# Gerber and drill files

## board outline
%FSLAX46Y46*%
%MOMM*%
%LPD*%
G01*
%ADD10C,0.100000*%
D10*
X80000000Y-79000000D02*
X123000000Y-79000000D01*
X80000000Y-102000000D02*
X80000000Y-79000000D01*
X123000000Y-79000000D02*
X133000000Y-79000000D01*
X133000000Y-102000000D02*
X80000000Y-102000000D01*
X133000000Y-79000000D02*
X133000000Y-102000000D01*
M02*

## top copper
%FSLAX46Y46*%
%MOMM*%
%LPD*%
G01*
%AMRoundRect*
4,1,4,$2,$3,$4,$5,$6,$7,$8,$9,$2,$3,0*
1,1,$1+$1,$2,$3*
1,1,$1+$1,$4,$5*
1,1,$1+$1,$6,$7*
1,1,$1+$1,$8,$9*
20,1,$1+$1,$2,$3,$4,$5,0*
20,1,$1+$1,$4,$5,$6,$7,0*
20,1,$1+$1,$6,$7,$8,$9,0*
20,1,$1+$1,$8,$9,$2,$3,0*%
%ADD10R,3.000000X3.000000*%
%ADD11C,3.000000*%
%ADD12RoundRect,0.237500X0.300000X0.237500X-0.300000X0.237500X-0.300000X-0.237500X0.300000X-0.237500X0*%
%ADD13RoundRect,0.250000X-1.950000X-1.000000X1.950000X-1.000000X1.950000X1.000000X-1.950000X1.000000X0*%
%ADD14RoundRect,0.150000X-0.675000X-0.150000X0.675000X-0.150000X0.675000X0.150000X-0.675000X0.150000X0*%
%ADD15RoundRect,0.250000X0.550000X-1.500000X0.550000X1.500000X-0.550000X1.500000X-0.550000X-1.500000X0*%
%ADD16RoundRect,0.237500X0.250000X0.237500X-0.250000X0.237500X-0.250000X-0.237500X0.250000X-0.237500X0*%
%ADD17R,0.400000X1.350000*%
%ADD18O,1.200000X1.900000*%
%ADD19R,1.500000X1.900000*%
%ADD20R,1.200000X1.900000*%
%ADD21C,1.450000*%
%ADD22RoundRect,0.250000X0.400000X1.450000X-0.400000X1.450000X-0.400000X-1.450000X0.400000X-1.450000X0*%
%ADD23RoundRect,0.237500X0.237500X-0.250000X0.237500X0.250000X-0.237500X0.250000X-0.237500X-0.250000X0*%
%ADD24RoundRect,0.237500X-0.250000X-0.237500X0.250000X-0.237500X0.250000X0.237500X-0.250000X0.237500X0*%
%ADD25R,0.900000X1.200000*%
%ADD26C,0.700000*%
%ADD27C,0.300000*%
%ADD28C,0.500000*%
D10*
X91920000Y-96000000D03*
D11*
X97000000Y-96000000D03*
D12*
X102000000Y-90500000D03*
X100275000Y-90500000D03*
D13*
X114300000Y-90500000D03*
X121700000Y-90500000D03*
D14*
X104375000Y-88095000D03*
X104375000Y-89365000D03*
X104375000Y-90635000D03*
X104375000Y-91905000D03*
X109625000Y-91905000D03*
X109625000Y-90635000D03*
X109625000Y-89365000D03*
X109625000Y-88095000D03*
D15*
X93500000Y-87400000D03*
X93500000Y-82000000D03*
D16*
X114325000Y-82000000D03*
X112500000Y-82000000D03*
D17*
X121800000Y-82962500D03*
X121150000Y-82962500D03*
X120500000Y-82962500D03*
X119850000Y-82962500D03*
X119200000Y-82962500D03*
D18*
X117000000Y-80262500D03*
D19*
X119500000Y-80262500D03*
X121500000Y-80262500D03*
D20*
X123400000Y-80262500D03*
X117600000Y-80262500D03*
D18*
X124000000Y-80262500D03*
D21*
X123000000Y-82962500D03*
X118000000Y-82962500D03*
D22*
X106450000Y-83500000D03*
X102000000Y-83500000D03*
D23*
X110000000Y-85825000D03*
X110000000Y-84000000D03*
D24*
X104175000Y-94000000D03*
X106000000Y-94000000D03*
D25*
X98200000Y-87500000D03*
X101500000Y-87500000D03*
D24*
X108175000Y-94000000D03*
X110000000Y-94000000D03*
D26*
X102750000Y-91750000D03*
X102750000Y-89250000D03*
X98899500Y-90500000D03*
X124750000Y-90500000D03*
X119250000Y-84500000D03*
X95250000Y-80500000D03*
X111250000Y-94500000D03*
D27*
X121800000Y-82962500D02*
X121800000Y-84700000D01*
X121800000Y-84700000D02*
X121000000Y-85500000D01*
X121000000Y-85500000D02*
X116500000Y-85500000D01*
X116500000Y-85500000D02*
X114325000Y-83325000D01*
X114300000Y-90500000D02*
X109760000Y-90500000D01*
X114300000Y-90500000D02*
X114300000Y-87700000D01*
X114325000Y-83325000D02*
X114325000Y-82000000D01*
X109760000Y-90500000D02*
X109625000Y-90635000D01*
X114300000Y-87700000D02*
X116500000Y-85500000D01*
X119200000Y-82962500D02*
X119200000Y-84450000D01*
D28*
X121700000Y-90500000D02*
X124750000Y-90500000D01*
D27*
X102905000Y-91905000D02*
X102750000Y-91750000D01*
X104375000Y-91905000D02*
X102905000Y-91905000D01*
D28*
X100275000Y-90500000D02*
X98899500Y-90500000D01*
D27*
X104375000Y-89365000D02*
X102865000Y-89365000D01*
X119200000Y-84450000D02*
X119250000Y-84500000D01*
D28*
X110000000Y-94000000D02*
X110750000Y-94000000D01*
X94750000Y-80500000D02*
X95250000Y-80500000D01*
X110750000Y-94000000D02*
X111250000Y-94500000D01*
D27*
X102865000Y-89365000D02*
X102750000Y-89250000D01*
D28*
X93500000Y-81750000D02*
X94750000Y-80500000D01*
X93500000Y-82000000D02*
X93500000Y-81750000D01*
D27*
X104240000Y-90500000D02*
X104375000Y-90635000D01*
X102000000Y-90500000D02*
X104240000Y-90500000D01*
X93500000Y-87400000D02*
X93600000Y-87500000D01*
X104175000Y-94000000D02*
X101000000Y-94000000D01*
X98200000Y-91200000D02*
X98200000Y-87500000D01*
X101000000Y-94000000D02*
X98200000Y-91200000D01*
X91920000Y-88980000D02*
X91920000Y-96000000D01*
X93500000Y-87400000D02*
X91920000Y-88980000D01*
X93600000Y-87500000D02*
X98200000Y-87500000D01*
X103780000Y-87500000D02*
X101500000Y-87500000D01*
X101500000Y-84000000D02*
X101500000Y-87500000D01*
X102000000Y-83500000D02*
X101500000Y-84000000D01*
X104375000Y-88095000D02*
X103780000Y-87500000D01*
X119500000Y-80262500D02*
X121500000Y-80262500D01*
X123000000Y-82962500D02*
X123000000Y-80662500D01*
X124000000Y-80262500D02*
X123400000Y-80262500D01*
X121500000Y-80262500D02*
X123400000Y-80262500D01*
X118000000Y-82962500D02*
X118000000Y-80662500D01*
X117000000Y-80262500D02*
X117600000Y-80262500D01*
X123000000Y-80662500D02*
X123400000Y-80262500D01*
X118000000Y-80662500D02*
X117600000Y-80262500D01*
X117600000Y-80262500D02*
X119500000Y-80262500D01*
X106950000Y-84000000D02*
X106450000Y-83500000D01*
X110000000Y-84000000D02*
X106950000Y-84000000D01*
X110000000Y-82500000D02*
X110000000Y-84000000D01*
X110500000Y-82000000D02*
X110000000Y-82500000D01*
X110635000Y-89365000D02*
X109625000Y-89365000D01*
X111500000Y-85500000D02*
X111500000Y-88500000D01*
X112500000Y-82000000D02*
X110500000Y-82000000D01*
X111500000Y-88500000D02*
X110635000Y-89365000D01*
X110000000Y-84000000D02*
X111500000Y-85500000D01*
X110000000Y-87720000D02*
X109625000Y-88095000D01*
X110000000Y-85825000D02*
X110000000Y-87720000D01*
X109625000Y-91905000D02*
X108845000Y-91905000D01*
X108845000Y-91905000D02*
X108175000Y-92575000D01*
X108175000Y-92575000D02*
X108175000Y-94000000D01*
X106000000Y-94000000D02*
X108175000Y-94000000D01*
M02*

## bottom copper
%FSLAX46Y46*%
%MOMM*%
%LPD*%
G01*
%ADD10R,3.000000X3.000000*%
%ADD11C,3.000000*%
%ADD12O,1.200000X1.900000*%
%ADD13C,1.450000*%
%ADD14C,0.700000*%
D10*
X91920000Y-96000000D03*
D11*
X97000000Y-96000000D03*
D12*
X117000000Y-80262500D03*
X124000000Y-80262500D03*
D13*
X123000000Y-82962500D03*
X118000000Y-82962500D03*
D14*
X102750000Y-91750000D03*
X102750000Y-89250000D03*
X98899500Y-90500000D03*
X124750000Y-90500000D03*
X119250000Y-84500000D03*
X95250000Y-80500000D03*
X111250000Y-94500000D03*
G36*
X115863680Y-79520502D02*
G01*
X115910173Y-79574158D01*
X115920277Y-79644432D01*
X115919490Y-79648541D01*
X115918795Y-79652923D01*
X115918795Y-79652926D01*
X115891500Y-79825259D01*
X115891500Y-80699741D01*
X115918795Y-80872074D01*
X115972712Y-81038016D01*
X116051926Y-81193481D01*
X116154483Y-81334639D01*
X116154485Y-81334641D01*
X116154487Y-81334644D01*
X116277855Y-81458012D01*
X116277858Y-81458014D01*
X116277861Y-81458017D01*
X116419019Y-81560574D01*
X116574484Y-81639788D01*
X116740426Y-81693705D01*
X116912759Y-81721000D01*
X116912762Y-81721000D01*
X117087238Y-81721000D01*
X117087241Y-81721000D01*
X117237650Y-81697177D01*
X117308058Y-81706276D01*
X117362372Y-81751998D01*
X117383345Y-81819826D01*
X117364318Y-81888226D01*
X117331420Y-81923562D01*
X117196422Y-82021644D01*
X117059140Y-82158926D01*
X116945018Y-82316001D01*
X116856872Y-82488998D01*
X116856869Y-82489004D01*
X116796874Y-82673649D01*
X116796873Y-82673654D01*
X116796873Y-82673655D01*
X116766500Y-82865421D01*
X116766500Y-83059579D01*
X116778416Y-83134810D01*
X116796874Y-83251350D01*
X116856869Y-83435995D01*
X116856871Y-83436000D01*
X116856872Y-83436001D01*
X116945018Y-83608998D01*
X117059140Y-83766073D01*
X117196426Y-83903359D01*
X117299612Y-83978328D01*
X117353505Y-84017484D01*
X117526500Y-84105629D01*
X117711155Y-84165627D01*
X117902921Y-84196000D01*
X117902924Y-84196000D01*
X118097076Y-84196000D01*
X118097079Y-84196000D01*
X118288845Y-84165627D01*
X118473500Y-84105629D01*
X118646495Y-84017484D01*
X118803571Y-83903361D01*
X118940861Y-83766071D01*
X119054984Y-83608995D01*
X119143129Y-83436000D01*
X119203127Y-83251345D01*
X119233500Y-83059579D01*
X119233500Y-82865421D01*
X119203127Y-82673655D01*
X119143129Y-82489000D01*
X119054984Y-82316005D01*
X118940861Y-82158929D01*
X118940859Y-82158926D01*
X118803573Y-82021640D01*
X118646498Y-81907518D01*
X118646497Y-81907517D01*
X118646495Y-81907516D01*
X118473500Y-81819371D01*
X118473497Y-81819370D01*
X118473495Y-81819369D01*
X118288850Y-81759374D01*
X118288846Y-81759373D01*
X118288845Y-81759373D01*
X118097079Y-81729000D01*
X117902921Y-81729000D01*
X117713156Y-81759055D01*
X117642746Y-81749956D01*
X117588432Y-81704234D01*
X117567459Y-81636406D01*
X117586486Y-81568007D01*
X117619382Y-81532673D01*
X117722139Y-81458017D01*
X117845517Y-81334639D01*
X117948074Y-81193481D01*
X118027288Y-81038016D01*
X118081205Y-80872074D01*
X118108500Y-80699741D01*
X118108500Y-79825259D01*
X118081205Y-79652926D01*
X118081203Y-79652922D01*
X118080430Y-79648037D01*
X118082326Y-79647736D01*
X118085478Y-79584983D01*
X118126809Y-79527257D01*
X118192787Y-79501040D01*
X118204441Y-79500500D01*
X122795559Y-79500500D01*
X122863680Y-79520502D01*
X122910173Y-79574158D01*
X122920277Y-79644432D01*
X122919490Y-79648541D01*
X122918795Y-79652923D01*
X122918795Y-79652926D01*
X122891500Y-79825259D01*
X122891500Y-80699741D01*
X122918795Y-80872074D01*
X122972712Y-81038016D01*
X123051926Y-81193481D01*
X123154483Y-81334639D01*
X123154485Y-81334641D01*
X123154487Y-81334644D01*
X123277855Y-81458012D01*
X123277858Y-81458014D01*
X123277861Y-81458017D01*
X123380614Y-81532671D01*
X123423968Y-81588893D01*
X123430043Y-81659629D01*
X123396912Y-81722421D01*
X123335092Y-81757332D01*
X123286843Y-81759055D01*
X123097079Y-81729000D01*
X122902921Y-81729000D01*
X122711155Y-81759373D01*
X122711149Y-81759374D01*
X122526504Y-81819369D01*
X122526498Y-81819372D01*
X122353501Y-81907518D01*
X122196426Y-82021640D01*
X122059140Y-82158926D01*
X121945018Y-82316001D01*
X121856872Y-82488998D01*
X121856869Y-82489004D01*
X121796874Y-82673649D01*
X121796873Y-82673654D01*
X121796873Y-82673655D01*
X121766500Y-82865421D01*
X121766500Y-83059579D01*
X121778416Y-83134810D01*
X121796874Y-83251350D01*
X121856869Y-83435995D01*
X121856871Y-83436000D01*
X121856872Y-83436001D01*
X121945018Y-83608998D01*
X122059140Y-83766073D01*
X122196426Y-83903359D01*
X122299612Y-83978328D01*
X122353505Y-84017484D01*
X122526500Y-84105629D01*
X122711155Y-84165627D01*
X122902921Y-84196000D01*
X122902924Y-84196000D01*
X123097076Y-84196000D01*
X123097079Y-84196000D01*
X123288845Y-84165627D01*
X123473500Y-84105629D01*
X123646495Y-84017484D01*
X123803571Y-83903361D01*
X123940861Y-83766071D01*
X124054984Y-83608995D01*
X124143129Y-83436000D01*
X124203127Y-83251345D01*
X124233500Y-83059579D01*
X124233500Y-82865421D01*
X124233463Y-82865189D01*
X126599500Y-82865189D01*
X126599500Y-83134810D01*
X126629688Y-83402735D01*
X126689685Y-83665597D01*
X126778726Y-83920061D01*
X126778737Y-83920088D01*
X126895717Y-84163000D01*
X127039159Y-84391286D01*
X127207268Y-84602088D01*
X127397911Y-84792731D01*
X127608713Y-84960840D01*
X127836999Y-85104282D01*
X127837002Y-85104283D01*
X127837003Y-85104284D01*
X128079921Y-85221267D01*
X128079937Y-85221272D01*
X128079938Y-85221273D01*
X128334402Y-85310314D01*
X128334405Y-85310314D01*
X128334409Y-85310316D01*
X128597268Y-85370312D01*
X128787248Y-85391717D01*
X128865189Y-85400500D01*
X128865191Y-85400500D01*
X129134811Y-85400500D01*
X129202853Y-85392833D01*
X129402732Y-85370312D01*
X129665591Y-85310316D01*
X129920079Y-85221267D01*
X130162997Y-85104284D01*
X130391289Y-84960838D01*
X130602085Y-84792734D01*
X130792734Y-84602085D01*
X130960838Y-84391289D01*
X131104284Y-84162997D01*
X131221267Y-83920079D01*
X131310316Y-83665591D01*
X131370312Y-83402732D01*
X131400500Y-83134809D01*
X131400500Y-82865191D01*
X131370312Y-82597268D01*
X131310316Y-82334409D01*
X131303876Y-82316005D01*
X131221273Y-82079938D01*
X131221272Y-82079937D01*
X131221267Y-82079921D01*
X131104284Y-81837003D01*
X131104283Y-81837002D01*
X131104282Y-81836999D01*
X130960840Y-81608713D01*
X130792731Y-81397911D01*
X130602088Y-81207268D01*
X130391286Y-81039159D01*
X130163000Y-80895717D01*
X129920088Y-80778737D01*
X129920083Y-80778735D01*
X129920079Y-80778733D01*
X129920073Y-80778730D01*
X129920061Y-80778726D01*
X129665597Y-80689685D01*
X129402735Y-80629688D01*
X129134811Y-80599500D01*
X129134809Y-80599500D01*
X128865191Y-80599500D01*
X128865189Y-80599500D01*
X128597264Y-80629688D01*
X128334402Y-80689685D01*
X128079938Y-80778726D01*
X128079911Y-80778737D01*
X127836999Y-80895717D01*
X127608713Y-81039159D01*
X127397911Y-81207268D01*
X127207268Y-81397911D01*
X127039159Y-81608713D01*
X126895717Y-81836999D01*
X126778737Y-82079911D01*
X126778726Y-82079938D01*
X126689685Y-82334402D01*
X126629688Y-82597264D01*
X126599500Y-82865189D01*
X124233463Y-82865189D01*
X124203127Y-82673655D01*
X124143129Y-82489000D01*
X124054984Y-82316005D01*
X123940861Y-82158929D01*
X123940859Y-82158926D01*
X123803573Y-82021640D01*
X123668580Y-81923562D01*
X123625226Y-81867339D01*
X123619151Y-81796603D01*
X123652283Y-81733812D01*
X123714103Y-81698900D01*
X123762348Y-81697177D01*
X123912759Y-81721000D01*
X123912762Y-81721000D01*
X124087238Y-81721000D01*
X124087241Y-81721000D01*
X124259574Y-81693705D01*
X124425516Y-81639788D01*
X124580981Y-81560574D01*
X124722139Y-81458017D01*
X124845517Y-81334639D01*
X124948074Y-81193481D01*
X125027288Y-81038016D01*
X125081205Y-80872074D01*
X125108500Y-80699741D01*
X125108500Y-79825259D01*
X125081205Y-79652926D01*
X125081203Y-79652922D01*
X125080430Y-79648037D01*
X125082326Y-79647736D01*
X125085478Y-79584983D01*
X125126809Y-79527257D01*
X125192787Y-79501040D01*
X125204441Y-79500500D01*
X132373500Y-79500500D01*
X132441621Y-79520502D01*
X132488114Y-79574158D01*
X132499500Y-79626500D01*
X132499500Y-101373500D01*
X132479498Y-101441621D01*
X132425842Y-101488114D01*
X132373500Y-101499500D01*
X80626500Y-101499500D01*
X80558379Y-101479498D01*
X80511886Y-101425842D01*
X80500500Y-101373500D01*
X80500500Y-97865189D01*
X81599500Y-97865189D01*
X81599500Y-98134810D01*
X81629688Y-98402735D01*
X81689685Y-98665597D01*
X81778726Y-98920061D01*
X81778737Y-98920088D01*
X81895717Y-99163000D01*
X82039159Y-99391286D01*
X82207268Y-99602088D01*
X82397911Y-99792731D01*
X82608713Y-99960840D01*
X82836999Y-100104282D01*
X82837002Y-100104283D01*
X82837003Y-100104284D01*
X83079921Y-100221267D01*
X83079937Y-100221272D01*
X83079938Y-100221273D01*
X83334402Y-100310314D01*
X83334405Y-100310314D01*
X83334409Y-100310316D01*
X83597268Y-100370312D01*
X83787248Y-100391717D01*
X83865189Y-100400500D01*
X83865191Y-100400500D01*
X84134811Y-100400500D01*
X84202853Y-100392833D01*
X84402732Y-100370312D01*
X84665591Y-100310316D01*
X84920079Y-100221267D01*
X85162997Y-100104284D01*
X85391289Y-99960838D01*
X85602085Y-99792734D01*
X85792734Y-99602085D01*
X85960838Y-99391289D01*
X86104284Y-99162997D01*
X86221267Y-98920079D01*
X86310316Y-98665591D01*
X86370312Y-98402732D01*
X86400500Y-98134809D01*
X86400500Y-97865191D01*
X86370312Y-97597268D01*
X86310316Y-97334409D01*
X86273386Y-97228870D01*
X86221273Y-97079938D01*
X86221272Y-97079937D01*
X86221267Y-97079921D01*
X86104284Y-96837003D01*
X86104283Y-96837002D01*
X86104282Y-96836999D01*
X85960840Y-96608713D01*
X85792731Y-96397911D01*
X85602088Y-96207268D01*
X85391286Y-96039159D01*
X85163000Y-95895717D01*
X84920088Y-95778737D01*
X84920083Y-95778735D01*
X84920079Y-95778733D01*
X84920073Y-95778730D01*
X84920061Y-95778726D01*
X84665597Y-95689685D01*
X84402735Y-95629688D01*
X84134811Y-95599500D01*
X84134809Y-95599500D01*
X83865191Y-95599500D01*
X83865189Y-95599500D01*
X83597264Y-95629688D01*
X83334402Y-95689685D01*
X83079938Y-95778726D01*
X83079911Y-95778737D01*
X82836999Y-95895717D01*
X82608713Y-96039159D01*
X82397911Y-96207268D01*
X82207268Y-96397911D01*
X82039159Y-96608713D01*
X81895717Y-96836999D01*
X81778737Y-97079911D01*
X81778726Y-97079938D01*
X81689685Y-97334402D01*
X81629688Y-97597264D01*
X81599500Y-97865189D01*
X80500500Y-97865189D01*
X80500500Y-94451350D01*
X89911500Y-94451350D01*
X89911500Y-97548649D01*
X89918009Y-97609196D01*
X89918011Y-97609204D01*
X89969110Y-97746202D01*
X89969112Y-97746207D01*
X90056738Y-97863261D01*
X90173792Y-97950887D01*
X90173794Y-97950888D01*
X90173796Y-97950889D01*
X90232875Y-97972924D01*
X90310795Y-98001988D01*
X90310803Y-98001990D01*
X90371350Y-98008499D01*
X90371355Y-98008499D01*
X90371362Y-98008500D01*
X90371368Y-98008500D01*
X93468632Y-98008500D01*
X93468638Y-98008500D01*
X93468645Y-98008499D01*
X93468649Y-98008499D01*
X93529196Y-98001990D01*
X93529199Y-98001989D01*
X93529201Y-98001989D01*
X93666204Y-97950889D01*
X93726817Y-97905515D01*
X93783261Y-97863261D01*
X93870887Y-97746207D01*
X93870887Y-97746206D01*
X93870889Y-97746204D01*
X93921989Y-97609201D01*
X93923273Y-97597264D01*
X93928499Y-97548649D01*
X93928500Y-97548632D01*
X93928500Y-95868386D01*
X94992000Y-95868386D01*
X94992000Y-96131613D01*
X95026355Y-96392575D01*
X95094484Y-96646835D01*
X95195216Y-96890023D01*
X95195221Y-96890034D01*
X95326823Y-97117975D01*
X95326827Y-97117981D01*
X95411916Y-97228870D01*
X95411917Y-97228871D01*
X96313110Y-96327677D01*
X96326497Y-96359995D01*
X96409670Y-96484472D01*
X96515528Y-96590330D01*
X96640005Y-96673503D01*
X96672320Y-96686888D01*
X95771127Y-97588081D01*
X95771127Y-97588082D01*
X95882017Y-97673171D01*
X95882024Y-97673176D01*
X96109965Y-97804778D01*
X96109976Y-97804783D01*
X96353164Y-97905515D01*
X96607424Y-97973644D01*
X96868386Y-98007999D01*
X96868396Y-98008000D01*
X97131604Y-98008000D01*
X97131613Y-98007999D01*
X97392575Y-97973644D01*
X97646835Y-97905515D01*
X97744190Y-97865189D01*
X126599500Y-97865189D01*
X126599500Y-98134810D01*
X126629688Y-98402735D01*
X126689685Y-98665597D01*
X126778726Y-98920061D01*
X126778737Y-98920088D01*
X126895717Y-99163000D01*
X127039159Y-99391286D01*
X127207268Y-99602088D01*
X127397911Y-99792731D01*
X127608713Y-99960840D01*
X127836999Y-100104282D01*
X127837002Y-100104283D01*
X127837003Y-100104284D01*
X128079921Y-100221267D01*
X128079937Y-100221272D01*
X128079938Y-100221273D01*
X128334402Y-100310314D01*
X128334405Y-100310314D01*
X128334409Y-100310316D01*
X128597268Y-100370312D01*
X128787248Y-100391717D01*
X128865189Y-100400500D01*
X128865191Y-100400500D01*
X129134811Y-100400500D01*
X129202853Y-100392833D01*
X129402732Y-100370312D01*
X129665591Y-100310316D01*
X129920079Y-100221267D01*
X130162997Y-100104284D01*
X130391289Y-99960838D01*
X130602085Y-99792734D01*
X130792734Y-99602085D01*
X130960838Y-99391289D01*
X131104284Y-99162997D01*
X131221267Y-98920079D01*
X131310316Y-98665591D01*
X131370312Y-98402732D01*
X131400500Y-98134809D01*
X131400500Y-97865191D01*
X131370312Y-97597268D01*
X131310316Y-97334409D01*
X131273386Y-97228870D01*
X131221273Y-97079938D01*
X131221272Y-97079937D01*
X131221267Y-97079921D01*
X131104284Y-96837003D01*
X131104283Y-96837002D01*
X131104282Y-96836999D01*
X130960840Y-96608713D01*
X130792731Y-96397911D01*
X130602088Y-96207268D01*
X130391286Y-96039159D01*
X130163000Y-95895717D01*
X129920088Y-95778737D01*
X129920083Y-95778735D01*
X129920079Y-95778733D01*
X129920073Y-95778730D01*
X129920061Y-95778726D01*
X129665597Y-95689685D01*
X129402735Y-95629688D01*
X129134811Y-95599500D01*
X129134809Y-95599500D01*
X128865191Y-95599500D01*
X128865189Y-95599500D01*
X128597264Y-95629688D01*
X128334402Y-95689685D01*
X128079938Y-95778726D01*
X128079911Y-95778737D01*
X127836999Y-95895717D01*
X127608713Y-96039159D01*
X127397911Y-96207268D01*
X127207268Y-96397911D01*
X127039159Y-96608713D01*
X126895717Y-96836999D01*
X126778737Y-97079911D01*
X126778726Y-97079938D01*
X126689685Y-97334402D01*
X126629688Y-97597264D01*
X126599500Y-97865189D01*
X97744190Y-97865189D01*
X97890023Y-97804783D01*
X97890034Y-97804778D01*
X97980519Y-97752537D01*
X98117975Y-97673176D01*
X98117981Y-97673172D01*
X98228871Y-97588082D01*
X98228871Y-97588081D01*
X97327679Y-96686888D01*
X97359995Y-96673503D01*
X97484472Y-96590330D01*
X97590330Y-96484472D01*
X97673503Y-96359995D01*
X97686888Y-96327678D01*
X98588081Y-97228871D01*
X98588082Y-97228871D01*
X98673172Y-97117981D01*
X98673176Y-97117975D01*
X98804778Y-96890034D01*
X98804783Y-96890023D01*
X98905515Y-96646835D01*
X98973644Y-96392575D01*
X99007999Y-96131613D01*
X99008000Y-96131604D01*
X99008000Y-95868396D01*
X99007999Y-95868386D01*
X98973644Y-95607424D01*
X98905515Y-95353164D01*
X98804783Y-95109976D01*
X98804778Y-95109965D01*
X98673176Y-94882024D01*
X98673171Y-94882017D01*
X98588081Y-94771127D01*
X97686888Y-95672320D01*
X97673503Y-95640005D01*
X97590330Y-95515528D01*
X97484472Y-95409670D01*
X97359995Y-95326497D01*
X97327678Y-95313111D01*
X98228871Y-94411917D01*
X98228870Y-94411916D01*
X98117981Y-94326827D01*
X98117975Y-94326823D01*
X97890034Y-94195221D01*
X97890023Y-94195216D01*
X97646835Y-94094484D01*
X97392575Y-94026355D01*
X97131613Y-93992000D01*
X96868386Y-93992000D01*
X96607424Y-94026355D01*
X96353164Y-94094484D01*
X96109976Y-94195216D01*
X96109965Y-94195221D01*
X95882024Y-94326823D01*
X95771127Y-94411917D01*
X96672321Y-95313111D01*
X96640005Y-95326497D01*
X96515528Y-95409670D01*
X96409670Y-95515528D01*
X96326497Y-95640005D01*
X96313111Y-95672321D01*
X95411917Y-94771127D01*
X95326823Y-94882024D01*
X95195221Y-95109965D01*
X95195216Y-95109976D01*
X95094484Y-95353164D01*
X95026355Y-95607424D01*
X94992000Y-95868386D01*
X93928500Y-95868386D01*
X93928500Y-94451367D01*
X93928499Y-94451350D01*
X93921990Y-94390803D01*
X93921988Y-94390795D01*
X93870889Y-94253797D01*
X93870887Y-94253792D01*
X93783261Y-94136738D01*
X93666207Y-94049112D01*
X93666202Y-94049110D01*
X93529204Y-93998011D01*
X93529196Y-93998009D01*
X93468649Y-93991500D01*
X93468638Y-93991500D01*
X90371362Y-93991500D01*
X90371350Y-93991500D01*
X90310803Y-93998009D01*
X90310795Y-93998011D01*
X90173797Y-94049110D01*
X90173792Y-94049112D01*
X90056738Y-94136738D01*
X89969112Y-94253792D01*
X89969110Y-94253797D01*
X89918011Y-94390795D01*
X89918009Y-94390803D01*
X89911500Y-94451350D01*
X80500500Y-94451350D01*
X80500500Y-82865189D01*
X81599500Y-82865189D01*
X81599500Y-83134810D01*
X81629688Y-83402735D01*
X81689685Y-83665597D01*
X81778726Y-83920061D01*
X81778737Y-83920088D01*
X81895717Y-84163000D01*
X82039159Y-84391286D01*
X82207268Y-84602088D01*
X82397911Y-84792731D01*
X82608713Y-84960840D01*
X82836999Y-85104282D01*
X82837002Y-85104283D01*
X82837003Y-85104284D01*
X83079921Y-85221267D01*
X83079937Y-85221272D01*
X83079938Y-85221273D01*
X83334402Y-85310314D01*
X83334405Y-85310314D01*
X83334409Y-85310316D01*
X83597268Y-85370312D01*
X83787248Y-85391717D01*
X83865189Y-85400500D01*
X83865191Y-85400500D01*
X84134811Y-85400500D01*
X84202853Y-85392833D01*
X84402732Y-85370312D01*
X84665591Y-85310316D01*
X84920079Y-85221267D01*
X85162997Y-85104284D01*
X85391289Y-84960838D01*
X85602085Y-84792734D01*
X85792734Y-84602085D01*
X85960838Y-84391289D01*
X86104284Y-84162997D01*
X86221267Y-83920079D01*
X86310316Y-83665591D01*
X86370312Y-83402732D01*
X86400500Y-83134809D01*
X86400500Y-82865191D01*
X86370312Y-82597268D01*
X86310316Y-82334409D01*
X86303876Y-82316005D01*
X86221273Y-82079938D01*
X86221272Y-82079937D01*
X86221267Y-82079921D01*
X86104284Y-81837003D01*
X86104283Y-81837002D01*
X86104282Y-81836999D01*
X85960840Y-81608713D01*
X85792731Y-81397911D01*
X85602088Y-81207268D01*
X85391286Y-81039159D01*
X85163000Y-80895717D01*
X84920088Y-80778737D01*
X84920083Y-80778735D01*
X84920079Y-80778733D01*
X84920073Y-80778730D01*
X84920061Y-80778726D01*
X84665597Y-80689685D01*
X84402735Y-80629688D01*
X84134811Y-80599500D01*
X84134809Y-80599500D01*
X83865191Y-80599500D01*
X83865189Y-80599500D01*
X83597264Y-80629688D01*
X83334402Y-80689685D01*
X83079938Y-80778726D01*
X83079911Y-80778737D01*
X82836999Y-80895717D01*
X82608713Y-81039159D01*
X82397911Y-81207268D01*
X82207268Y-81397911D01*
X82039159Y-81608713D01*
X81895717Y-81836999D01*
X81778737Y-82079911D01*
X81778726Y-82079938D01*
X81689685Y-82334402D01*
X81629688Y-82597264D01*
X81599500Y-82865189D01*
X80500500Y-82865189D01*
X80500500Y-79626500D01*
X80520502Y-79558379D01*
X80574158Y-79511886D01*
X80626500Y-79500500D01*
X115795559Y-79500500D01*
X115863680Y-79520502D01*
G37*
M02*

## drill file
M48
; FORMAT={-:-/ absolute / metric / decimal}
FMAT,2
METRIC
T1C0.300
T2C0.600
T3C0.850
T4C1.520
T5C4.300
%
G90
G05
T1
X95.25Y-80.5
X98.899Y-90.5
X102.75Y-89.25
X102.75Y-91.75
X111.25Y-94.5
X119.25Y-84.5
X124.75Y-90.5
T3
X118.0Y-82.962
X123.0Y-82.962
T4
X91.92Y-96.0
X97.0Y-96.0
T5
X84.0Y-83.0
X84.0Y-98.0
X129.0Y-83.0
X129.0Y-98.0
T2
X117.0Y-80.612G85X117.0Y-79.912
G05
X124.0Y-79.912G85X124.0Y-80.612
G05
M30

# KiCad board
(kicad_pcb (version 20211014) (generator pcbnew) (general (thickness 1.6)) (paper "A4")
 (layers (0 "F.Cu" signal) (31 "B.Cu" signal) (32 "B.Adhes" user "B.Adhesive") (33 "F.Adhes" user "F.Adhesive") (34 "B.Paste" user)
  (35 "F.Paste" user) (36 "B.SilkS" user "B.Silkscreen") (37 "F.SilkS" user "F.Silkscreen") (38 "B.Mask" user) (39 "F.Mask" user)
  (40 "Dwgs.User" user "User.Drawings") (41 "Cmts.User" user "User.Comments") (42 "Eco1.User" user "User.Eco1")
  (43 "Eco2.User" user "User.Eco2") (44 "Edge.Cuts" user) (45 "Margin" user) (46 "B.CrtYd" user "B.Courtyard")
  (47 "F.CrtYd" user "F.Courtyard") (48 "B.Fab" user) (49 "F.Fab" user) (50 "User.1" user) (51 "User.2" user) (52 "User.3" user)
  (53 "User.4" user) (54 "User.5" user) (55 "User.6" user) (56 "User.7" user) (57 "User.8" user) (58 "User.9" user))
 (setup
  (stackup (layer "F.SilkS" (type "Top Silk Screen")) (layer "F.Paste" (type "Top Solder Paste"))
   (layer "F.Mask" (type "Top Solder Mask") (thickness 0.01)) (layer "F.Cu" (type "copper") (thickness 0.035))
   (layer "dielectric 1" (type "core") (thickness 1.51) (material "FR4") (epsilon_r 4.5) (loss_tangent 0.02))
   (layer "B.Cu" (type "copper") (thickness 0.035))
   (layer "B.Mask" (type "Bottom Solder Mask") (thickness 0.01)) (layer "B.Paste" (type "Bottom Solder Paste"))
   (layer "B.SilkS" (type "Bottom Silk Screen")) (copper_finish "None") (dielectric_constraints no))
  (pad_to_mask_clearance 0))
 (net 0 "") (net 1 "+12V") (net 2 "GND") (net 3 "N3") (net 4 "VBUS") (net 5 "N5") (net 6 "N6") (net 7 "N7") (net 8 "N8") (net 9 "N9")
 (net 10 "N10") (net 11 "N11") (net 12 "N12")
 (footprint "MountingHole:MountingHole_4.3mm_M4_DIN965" (layer "F.Cu") (at 84 83)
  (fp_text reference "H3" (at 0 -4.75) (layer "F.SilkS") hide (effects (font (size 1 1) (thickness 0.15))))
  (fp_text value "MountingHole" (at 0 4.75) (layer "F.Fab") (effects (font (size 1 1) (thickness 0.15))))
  (pad "" np_thru_hole circle (at 0 0) (size 4.3 4.3) (drill 4.3) (layers *.Cu *.Mask)))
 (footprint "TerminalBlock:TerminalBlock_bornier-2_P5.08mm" (layer "F.Cu") (at 91.92 96)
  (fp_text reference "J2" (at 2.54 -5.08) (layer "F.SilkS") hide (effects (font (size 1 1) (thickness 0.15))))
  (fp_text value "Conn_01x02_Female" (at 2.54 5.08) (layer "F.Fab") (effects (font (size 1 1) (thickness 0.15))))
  (pad "1" thru_hole rect (at 0 0) (size 3 3) (drill 1.52) (layers *.Cu *.Mask) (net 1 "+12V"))
  (pad "2" thru_hole circle (at 5.08 0) (size 3 3) (drill 1.52) (layers *.Cu *.Mask) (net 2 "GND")))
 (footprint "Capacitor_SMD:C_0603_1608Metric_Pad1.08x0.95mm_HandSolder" (layer "F.Cu") (at 101.1375 90.5 180)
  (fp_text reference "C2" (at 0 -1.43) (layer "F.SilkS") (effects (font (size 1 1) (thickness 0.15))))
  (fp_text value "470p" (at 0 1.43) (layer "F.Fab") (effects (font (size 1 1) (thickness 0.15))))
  (pad "1" smd roundrect (at -0.8625 0 180) (size 1.075 0.95) (layers "F.Cu" "F.Paste" "F.Mask") (roundrect_rratio 0.25) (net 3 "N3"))
  (pad "2" smd roundrect (at 0.8625 0 180) (size 1.075 0.95) (layers "F.Cu" "F.Paste" "F.Mask") (roundrect_rratio 0.25) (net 2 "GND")))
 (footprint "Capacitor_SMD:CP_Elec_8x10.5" (layer "F.Cu") (at 118 90.5)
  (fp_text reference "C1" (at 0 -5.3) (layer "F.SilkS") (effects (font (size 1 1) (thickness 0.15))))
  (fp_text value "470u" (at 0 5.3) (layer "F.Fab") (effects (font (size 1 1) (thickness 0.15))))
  (pad "1" smd roundrect (at -3.7 0) (size 4.4 2.5) (layers "F.Cu" "F.Paste" "F.Mask") (roundrect_rratio 0.1) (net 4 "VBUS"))
  (pad "2" smd roundrect (at 3.7 0) (size 4.4 2.5) (layers "F.Cu" "F.Paste" "F.Mask") (roundrect_rratio 0.1) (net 2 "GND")))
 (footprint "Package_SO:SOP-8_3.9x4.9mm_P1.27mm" (layer "F.Cu") (at 107 90)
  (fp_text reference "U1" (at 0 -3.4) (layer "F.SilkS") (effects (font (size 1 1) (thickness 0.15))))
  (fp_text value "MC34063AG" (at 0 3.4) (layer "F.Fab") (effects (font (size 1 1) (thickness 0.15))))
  (pad "1" smd roundrect (at -2.625 -1.905) (size 1.65 0.6) (layers "F.Cu" "F.Paste" "F.Mask") (roundrect_rratio 0.25) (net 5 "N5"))
  (pad "2" smd roundrect (at -2.625 -0.635) (size 1.65 0.6) (layers "F.Cu" "F.Paste" "F.Mask") (roundrect_rratio 0.25) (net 2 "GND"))
  (pad "3" smd roundrect (at -2.625 0.635) (size 1.65 0.6) (layers "F.Cu" "F.Paste" "F.Mask") (roundrect_rratio 0.25) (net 3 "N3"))
  (pad "4" smd roundrect (at -2.625 1.905) (size 1.65 0.6) (layers "F.Cu" "F.Paste" "F.Mask") (roundrect_rratio 0.25) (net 2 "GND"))
  (pad "5" smd roundrect (at 2.625 1.905) (size 1.65 0.6) (layers "F.Cu" "F.Paste" "F.Mask") (roundrect_rratio 0.25) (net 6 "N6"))
  (pad "6" smd roundrect (at 2.625 0.635) (size 1.65 0.6) (layers "F.Cu" "F.Paste" "F.Mask") (roundrect_rratio 0.25) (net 4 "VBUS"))
  (pad "7" smd roundrect (at 2.625 -0.635) (size 1.65 0.6) (layers "F.Cu" "F.Paste" "F.Mask") (roundrect_rratio 0.25) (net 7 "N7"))
  (pad "8" smd roundrect (at 2.625 -1.905) (size 1.65 0.6) (layers "F.Cu" "F.Paste" "F.Mask") (roundrect_rratio 0.25) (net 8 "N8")))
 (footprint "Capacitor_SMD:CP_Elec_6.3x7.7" (layer "F.Cu") (at 93.5 84.7 90)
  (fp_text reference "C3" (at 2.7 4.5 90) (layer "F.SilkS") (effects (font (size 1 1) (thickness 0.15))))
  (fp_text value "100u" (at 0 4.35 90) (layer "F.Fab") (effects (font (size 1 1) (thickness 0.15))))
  (pad "1" smd roundrect (at -2.7 0 90) (size 3.5 1.6) (layers "F.Cu" "F.Paste" "F.Mask") (roundrect_rratio 0.15625) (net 1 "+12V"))
  (pad "2" smd roundrect (at 2.7 0 90) (size 3.5 1.6) (layers "F.Cu" "F.Paste" "F.Mask") (roundrect_rratio 0.15625) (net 2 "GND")))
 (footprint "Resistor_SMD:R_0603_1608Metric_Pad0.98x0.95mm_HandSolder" (layer "F.Cu") (at 113.4125 82 180)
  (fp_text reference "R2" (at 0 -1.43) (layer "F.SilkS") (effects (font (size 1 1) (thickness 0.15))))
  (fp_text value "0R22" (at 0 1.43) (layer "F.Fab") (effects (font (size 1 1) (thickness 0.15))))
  (pad "1" smd roundrect (at -0.9125 0 180) (size 0.975 0.95) (layers "F.Cu" "F.Paste" "F.Mask") (roundrect_rratio 0.25) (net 4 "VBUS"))
  (pad "2" smd roundrect (at 0.9125 0 180) (size 0.975 0.95) (layers "F.Cu" "F.Paste" "F.Mask") (roundrect_rratio 0.25) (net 7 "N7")))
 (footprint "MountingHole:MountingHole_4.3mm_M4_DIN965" (layer "F.Cu") (at 84 98)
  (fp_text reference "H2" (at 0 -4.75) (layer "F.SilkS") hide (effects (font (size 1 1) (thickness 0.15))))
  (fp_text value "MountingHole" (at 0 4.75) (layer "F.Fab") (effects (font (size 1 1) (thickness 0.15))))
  (pad "" np_thru_hole circle (at 0 0) (size 4.3 4.3) (drill 4.3) (layers *.Cu *.Mask)))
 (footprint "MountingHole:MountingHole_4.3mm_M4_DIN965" (layer "F.Cu") (at 129 98)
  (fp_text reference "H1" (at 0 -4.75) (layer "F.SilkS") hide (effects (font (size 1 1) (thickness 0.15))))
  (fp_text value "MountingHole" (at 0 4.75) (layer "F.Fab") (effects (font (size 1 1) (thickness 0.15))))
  (pad "" np_thru_hole circle (at 0 0) (size 4.3 4.3) (drill 4.3) (layers *.Cu *.Mask)))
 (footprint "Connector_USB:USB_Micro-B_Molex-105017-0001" (layer "F.Cu") (at 120.5 81.5 180)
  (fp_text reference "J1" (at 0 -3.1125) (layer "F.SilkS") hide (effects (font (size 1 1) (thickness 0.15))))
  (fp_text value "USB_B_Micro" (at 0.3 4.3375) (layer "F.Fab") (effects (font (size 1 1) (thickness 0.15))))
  (pad "1" smd rect (at -1.3 -1.4625 180) (size 0.4 1.35) (layers "F.Cu" "F.Paste" "F.Mask") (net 4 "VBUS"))
  (pad "2" smd rect (at -0.65 -1.4625 180) (size 0.4 1.35) (layers "F.Cu" "F.Paste" "F.Mask") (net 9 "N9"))
  (pad "3" smd rect (at 0 -1.4625 180) (size 0.4 1.35) (layers "F.Cu" "F.Paste" "F.Mask") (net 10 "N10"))
  (pad "4" smd rect (at 0.65 -1.4625 180) (size 0.4 1.35) (layers "F.Cu" "F.Paste" "F.Mask") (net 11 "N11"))
  (pad "5" smd rect (at 1.3 -1.4625 180) (size 0.4 1.35) (layers "F.Cu" "F.Paste" "F.Mask") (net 2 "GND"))
  (pad "6" thru_hole oval (at 3.5 1.2375 180) (size 1.2 1.9) (drill oval 0.6 1.3) (layers *.Cu *.Mask) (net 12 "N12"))
  (pad "6" smd rect (at 1 1.2375 180) (size 1.5 1.9) (layers "F.Cu" "F.Paste" "F.Mask") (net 12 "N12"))
  (pad "6" smd rect (at -1 1.2375 180) (size 1.5 1.9) (layers "F.Cu" "F.Paste" "F.Mask") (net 12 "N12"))
  (pad "6" smd rect (at -2.9 1.2375 180) (size 1.2 1.9) (layers "F.Cu" "F.Mask") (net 12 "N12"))
  (pad "6" smd rect (at 2.9 1.2375 180) (size 1.2 1.9) (layers "F.Cu" "F.Mask") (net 12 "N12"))
  (pad "6" thru_hole oval (at -3.5 1.2375) (size 1.2 1.9) (drill oval 0.6 1.3) (layers *.Cu *.Mask) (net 12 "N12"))
  (pad "6" thru_hole circle (at -2.5 -1.4625 180) (size 1.45 1.45) (drill 0.85) (layers *.Cu *.Mask) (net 12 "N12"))
  (pad "6" thru_hole circle (at 2.5 -1.4625 180) (size 1.45 1.45) (drill 0.85) (layers *.Cu *.Mask) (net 12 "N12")))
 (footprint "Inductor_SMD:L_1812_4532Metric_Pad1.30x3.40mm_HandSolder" (layer "F.Cu") (at 104.225 83.5 180)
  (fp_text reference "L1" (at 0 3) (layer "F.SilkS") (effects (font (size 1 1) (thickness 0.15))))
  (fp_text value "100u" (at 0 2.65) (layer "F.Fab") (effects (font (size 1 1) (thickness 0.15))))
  (pad "1" smd roundrect (at -2.225 0 180) (size 1.3 3.4) (layers "F.Cu" "F.Paste" "F.Mask") (roundrect_rratio 0.1923076923) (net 7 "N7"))
  (pad "2" smd roundrect (at 2.225 0 180) (size 1.3 3.4) (layers "F.Cu" "F.Paste" "F.Mask") (roundrect_rratio 0.1923076923) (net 5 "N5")))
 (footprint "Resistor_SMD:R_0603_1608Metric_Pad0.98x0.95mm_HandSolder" (layer "F.Cu") (at 110 84.9125 90)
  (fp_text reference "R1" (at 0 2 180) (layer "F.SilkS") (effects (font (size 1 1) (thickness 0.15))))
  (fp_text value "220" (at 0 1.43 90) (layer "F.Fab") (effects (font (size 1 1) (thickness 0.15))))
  (pad "1" smd roundrect (at -0.9125 0 90) (size 0.975 0.95) (layers "F.Cu" "F.Paste" "F.Mask") (roundrect_rratio 0.25) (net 8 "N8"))
  (pad "2" smd roundrect (at 0.9125 0 90) (size 0.975 0.95) (layers "F.Cu" "F.Paste" "F.Mask") (roundrect_rratio 0.25) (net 7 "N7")))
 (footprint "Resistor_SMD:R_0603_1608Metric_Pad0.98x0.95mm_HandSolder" (layer "F.Cu") (at 105.0875 94)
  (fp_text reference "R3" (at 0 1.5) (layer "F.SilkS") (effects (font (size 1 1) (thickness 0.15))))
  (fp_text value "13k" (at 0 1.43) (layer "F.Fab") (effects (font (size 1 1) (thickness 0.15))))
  (pad "1" smd roundrect (at -0.9125 0) (size 0.975 0.95) (layers "F.Cu" "F.Paste" "F.Mask") (roundrect_rratio 0.25) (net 1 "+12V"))
  (pad "2" smd roundrect (at 0.9125 0) (size 0.975 0.95) (layers "F.Cu" "F.Paste" "F.Mask") (roundrect_rratio 0.25) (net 6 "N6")))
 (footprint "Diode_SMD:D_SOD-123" (layer "F.Cu") (at 99.85 87.5)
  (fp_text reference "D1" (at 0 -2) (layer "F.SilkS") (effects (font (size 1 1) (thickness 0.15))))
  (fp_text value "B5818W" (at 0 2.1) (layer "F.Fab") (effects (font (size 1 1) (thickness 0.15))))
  (pad "1" smd rect (at -1.65 0) (size 0.9 1.2) (layers "F.Cu" "F.Paste" "F.Mask") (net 1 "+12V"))
  (pad "2" smd rect (at 1.65 0) (size 0.9 1.2) (layers "F.Cu" "F.Paste" "F.Mask") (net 5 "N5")))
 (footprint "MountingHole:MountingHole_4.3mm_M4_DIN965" (layer "F.Cu") (at 129 83)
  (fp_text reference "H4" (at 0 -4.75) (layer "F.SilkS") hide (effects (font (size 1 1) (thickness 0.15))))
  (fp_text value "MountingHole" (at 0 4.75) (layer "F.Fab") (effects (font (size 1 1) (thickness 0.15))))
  (pad "" np_thru_hole circle (at 0 0) (size 4.3 4.3) (drill 4.3) (layers *.Cu *.Mask)))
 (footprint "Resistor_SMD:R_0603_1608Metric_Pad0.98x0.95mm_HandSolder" (layer "F.Cu") (at 109.0875 94)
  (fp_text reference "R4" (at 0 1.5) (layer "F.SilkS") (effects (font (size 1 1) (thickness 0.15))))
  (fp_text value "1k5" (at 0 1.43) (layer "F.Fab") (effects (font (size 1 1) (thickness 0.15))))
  (pad "1" smd roundrect (at -0.9125 0) (size 0.975 0.95) (layers "F.Cu" "F.Paste" "F.Mask") (roundrect_rratio 0.25) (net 6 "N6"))
  (pad "2" smd roundrect (at 0.9125 0) (size 0.975 0.95) (layers "F.Cu" "F.Paste" "F.Mask") (roundrect_rratio 0.25) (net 2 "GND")))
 (gr_line (start 80 79) (end 123 79) (layer "Edge.Cuts") (width 0.1))
 (gr_line (start 80 102) (end 80 79) (layer "Edge.Cuts") (width 0.1))
 (gr_line (start 123 79) (end 133 79) (layer "Edge.Cuts") (width 0.1))
 (gr_line (start 133 102) (end 80 102) (layer "Edge.Cuts") (width 0.1))
 (gr_line (start 133 79) (end 133 102) (layer "Edge.Cuts") (width 0.1))
 (segment (start 121.8 82.9625) (end 121.8 84.7) (width 0.3) (layer "F.Cu") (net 4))
 (segment (start 121.8 84.7) (end 121 85.5) (width 0.3) (layer "F.Cu") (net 4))
 (segment (start 121 85.5) (end 116.5 85.5) (width 0.3) (layer "F.Cu") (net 4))
 (segment (start 116.5 85.5) (end 114.325 83.325) (width 0.3) (layer "F.Cu") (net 4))
 (segment (start 114.3 90.5) (end 109.76 90.5) (width 0.3) (layer "F.Cu") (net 4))
 (segment (start 114.3 90.5) (end 114.3 87.7) (width 0.3) (layer "F.Cu") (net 4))
 (segment (start 114.325 83.325) (end 114.325 82) (width 0.3) (layer "F.Cu") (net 4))
 (segment (start 109.76 90.5) (end 109.625 90.635) (width 0.3) (layer "F.Cu") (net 4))
 (segment (start 114.3 87.7) (end 116.5 85.5) (width 0.3) (layer "F.Cu") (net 4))
 (segment (start 119.2 82.9625) (end 119.2 84.45) (width 0.3) (layer "F.Cu") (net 2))
 (segment (start 121.7 90.5) (end 124.75 90.5) (width 0.5) (layer "F.Cu") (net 2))
 (segment (start 102.905 91.905) (end 102.75 91.75) (width 0.3) (layer "F.Cu") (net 2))
 (segment (start 104.375 91.905) (end 102.905 91.905) (width 0.3) (layer "F.Cu") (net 2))
 (segment (start 100.275 90.5) (end 98.8995 90.5) (width 0.5) (layer "F.Cu") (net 2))
 (segment (start 104.375 89.365) (end 102.865 89.365) (width 0.3) (layer "F.Cu") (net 2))
 (segment (start 119.2 84.45) (end 119.25 84.5) (width 0.3) (layer "F.Cu") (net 2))
 (segment (start 110 94) (end 110.75 94) (width 0.5) (layer "F.Cu") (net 2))
 (segment (start 94.75 80.5) (end 95.25 80.5) (width 0.5) (layer "F.Cu") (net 2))
 (segment (start 110.75 94) (end 111.25 94.5) (width 0.5) (layer "F.Cu") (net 2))
 (segment (start 102.865 89.365) (end 102.75 89.25) (width 0.3) (layer "F.Cu") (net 2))
 (segment (start 93.5 81.75) (end 94.75 80.5) (width 0.5) (layer "F.Cu") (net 2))
 (segment (start 93.5 82) (end 93.5 81.75) (width 0.5) (layer "F.Cu") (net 2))
 (via (at 102.75 91.75) (size 0.7) (drill 0.3) (layers "F.Cu" "B.Cu") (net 2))
 (via (at 102.75 89.25) (size 0.7) (drill 0.3) (layers "F.Cu" "B.Cu") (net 2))
 (via (at 98.8995 90.5) (size 0.7) (drill 0.3) (layers "F.Cu" "B.Cu") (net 2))
 (via (at 124.75 90.5) (size 0.7) (drill 0.3) (layers "F.Cu" "B.Cu") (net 2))
 (via (at 119.25 84.5) (size 0.7) (drill 0.3) (layers "F.Cu" "B.Cu") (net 2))
 (via (at 95.25 80.5) (size 0.7) (drill 0.3) (layers "F.Cu" "B.Cu") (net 2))
 (via (at 111.25 94.5) (size 0.7) (drill 0.3) (layers "F.Cu" "B.Cu") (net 2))
 (segment (start 104.24 90.5) (end 104.375 90.635) (width 0.3) (layer "F.Cu") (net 3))
 (segment (start 102 90.5) (end 104.24 90.5) (width 0.3) (layer "F.Cu") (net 3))
 (segment (start 93.5 87.4) (end 93.6 87.5) (width 0.3) (layer "F.Cu") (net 1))
 (segment (start 104.175 94) (end 101 94) (width 0.3) (layer "F.Cu") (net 1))
 (segment (start 98.2 91.2) (end 98.2 87.5) (width 0.3) (layer "F.Cu") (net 1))
 (segment (start 101 94) (end 98.2 91.2) (width 0.3) (layer "F.Cu") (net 1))
 (segment (start 91.92 88.98) (end 91.92 96) (width 0.3) (layer "F.Cu") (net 1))
 (segment (start 93.5 87.4) (end 91.92 88.98) (width 0.3) (layer "F.Cu") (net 1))
 (segment (start 93.6 87.5) (end 98.2 87.5) (width 0.3) (layer "F.Cu") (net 1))
 (segment (start 103.78 87.5) (end 101.5 87.5) (width 0.3) (layer "F.Cu") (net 5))
 (segment (start 101.5 84) (end 101.5 87.5) (width 0.3) (layer "F.Cu") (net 5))
 (segment (start 102 83.5) (end 101.5 84) (width 0.3) (layer "F.Cu") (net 5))
 (segment (start 104.375 88.095) (end 103.78 87.5) (width 0.3) (layer "F.Cu") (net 5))
 (segment (start 119.5 80.2625) (end 121.5 80.2625) (width 0.3) (layer "F.Cu") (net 12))
 (segment (start 123 82.9625) (end 123 80.6625) (width 0.3) (layer "F.Cu") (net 12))
 (segment (start 124 80.2625) (end 123.4 80.2625) (width 0.3) (layer "F.Cu") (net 12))
 (segment (start 121.5 80.2625) (end 123.4 80.2625) (width 0.3) (layer "F.Cu") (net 12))
 (segment (start 118 82.9625) (end 118 80.6625) (width 0.3) (layer "F.Cu") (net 12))
 (segment (start 117 80.2625) (end 117.6 80.2625) (width 0.3) (layer "F.Cu") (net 12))
 (segment (start 123 80.6625) (end 123.4 80.2625) (width 0.3) (layer "F.Cu") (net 12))
 (segment (start 118 80.6625) (end 117.6 80.2625) (width 0.3) (layer "F.Cu") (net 12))
 (segment (start 117.6 80.2625) (end 119.5 80.2625) (width 0.3) (layer "F.Cu") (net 12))
 (segment (start 106.95 84) (end 106.45 83.5) (width 0.3) (layer "F.Cu") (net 7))
 (segment (start 110 84) (end 106.95 84) (width 0.3) (layer "F.Cu") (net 7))
 (segment (start 110 82.5) (end 110 84) (width 0.3) (layer "F.Cu") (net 7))
 (segment (start 110.5 82) (end 110 82.5) (width 0.3) (layer "F.Cu") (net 7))
 (segment (start 110.635 89.365) (end 109.625 89.365) (width 0.3) (layer "F.Cu") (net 7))
 (segment (start 111.5 85.5) (end 111.5 88.5) (width 0.3) (layer "F.Cu") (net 7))
 (segment (start 112.5 82) (end 110.5 82) (width 0.3) (layer "F.Cu") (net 7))
 (segment (start 111.5 88.5) (end 110.635 89.365) (width 0.3) (layer "F.Cu") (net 7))
 (segment (start 110 84) (end 111.5 85.5) (width 0.3) (layer "F.Cu") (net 7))
 (segment (start 110 87.72) (end 109.625 88.095) (width 0.3) (layer "F.Cu") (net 8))
 (segment (start 110 85.825) (end 110 87.72) (width 0.3) (layer "F.Cu") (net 8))
 (segment (start 109.625 91.905) (end 108.845 91.905) (width 0.3) (layer "F.Cu") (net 6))
 (segment (start 108.845 91.905) (end 108.175 92.575) (width 0.3) (layer "F.Cu") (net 6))
 (segment (start 108.175 92.575) (end 108.175 94) (width 0.3) (layer "F.Cu") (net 6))
 (segment (start 106 94) (end 108.175 94) (width 0.3) (layer "F.Cu") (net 6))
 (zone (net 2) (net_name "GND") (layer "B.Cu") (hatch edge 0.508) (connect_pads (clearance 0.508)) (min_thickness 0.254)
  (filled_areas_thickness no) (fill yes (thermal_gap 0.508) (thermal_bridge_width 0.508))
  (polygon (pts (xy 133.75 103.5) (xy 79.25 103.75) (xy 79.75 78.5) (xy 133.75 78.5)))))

